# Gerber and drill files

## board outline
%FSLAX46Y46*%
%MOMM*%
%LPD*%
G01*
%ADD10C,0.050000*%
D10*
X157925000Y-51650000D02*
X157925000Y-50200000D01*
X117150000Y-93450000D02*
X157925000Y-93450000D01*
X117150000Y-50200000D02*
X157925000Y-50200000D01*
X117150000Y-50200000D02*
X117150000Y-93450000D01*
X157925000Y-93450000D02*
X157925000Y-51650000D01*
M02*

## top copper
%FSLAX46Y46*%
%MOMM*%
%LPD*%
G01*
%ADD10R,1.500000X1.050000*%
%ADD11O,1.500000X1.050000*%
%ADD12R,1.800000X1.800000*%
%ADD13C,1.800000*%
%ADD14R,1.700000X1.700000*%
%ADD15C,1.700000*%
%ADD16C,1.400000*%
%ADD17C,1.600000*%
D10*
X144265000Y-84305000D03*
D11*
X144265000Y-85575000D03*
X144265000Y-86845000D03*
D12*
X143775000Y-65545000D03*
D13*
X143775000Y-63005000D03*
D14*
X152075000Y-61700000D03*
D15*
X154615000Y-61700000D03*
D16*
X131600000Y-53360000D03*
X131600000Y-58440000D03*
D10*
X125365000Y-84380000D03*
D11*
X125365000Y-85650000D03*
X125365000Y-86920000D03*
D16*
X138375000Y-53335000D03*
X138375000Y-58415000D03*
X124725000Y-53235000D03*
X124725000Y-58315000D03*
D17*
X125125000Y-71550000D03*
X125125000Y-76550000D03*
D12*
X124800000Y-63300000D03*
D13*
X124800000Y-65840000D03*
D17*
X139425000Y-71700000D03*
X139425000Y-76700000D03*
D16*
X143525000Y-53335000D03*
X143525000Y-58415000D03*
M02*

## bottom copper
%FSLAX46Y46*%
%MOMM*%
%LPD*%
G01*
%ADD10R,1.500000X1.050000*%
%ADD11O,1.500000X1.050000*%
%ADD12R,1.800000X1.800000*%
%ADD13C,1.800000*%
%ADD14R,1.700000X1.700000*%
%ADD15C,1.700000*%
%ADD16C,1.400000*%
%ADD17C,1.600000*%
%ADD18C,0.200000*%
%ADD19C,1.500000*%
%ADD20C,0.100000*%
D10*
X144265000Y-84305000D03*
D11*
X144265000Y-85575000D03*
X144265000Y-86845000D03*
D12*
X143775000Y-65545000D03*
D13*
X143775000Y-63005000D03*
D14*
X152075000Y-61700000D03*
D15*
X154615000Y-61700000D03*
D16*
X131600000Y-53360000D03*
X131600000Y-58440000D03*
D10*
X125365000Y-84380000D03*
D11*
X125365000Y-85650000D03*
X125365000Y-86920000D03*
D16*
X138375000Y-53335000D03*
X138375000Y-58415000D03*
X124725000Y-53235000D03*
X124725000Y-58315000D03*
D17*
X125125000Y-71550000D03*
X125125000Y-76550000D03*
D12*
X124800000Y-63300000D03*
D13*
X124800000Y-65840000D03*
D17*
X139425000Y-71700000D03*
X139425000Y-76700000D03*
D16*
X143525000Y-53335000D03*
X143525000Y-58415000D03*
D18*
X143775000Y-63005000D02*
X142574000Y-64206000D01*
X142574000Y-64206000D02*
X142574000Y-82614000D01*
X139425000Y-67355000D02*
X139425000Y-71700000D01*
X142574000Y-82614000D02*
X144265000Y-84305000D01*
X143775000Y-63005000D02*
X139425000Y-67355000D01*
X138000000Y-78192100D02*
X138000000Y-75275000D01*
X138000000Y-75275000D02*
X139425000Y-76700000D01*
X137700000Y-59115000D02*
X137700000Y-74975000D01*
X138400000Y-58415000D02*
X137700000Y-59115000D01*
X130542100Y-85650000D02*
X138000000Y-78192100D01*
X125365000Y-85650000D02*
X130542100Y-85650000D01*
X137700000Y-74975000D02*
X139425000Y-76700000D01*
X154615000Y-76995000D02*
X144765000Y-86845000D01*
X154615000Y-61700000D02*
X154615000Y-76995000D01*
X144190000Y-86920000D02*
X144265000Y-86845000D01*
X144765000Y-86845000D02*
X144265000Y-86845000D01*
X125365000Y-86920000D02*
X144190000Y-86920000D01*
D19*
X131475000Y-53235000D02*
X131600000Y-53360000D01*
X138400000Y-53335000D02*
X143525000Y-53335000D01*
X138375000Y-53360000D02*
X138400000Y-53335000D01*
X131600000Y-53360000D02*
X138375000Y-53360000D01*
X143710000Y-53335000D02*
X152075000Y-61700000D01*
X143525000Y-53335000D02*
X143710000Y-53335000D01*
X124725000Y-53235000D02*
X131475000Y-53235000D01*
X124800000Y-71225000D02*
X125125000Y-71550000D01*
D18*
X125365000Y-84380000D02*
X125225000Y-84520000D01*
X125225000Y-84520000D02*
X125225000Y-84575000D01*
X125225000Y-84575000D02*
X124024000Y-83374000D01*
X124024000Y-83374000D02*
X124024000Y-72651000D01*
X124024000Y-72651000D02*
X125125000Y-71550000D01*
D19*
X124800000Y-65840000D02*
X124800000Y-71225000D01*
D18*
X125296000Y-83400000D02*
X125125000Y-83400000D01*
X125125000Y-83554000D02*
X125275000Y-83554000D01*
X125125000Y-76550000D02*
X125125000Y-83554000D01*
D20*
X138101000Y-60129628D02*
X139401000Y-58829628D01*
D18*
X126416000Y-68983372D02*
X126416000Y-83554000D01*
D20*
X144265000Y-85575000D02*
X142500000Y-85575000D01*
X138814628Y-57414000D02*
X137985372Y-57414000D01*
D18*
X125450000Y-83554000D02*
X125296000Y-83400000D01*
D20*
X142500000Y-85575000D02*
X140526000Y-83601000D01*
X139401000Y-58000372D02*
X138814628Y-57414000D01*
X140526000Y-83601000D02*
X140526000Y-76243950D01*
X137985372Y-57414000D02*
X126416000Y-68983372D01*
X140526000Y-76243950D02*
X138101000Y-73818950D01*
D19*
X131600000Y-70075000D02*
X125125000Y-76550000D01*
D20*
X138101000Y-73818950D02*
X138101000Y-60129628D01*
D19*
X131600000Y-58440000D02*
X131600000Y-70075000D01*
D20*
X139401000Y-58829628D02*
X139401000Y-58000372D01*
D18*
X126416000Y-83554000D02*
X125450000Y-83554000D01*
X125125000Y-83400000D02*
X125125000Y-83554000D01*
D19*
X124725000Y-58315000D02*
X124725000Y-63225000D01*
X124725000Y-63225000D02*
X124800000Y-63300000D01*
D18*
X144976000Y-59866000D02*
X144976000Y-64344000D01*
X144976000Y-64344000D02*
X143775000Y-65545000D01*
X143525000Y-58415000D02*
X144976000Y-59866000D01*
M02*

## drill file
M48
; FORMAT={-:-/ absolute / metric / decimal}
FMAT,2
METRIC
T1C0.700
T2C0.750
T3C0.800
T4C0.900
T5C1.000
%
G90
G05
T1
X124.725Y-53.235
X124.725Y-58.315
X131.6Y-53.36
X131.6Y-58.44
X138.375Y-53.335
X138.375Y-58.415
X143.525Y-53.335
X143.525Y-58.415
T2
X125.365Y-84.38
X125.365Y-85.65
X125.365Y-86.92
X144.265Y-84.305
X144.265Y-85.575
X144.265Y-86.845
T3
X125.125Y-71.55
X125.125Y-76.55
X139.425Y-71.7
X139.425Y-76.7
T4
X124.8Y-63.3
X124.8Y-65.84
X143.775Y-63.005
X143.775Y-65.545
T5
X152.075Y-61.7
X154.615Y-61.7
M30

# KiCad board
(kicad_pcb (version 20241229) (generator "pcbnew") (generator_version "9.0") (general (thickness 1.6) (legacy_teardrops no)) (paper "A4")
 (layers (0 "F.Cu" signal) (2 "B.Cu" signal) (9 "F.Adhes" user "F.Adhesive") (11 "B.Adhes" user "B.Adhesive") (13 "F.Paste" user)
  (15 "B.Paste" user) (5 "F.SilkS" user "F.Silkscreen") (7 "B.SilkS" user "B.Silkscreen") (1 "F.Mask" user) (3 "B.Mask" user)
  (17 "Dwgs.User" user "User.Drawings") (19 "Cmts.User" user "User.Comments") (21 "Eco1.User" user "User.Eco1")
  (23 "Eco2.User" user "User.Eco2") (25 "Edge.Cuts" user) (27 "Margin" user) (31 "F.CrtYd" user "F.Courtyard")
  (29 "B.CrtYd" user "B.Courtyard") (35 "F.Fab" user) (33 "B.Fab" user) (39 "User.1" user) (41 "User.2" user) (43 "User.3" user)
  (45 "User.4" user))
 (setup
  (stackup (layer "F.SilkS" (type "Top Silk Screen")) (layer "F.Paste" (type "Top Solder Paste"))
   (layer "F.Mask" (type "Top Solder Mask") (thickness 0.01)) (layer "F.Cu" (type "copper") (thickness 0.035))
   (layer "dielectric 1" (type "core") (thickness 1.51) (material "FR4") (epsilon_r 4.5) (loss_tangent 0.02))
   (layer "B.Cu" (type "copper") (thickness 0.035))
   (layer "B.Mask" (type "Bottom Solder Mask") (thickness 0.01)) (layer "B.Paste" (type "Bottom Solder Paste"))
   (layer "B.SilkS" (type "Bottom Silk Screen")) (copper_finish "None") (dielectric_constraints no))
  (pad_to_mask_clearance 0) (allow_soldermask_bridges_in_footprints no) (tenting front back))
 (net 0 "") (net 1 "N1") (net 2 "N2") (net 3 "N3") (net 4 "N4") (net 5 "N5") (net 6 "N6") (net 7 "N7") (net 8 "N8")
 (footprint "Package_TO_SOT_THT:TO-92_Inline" (layer "F.Cu") (at 144.265 84.305 -90)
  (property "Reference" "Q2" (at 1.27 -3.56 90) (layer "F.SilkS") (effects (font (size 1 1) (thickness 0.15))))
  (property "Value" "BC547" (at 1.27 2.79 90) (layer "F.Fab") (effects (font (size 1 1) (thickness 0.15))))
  (pad "1" thru_hole rect (at 0 0 270) (size 1.05 1.5) (drill 0.75) (layers "*.Cu" "*.Mask") (remove_unused_layers no) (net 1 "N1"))
  (pad "2" thru_hole oval (at 1.27 0 270) (size 1.05 1.5) (drill 0.75) (layers "*.Cu" "*.Mask") (remove_unused_layers no) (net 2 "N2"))
  (pad "3" thru_hole oval (at 2.54 0 270) (size 1.05 1.5) (drill 0.75) (layers "*.Cu" "*.Mask") (remove_unused_layers no) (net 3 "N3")))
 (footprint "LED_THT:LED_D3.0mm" (layer "F.Cu") (at 143.775 65.545 90)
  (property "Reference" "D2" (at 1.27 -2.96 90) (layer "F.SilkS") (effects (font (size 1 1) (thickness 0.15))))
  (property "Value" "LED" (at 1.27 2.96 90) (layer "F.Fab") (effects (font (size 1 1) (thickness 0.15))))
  (pad "1" thru_hole rect (at 0 0 90) (size 1.8 1.8) (drill 0.9) (layers "*.Cu" "*.Mask") (remove_unused_layers no) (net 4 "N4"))
  (pad "2" thru_hole circle (at 2.54 0 90) (size 1.8 1.8) (drill 0.9) (layers "*.Cu" "*.Mask") (remove_unused_layers no) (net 1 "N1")))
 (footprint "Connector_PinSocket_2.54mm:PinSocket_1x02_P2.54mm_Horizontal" (layer "F.Cu") (at 152.075 61.7 90)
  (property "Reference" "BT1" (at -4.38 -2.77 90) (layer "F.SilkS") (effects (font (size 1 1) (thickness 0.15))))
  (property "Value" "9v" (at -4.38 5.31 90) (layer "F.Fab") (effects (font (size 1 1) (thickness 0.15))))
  (pad "1" thru_hole rect (at 0 0 90) (size 1.7 1.7) (drill 1) (layers "*.Cu" "*.Mask") (remove_unused_layers no) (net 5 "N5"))
  (pad "2" thru_hole circle (at 0 2.54 90) (size 1.7 1.7) (drill 1) (layers "*.Cu" "*.Mask") (remove_unused_layers no) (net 3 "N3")))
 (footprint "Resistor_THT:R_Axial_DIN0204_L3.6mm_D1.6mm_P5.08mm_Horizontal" (layer "F.Cu") (at 131.6 53.36 -90)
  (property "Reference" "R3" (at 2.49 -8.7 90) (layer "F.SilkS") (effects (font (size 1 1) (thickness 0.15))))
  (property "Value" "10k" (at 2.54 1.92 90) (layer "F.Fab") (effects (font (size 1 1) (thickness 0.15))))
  (pad "1" thru_hole circle (at 0 0 270) (size 1.4 1.4) (drill 0.7) (layers "*.Cu" "*.Mask") (remove_unused_layers no) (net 5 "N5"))
  (pad "2" thru_hole circle (at 5.08 0 270) (size 1.4 1.4) (drill 0.7) (layers "*.Cu" "*.Mask") (remove_unused_layers no) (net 2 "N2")))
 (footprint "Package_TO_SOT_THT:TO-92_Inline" (layer "F.Cu") (at 125.365 84.38 -90)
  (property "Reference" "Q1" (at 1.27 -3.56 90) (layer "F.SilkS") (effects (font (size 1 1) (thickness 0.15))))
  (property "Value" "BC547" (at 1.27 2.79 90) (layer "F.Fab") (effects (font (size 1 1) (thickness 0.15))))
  (pad "1" thru_hole rect (at 0 0 270) (size 1.05 1.5) (drill 0.75) (layers "*.Cu" "*.Mask") (remove_unused_layers no) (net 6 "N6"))
  (pad "2" thru_hole oval (at 1.27 0 270) (size 1.05 1.5) (drill 0.75) (layers "*.Cu" "*.Mask") (remove_unused_layers no) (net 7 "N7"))
  (pad "3" thru_hole oval (at 2.54 0 270) (size 1.05 1.5) (drill 0.75) (layers "*.Cu" "*.Mask") (remove_unused_layers no) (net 3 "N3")))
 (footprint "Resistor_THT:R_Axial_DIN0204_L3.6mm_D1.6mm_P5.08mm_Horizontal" (layer "F.Cu") (at 138.375 53.335 -90)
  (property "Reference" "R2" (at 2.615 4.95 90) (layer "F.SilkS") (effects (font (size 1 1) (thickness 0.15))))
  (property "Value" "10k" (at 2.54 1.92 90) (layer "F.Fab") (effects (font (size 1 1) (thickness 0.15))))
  (pad "1" thru_hole circle (at 0 0 270) (size 1.4 1.4) (drill 0.7) (layers "*.Cu" "*.Mask") (remove_unused_layers no) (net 5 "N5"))
  (pad "2" thru_hole circle (at 5.08 0 270) (size 1.4 1.4) (drill 0.7) (layers "*.Cu" "*.Mask") (remove_unused_layers no) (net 7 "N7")))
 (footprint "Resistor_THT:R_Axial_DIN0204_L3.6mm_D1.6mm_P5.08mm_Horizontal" (layer "F.Cu") (at 124.725 53.235 -90)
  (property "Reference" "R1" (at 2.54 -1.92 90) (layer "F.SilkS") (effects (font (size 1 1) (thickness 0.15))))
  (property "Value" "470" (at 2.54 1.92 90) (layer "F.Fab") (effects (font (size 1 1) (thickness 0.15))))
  (pad "1" thru_hole circle (at 0 0 270) (size 1.4 1.4) (drill 0.7) (layers "*.Cu" "*.Mask") (remove_unused_layers no) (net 5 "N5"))
  (pad "2" thru_hole circle (at 5.08 0 270) (size 1.4 1.4) (drill 0.7) (layers "*.Cu" "*.Mask") (remove_unused_layers no) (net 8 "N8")))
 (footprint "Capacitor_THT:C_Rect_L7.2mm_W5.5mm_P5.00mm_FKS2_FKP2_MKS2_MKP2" (layer "F.Cu") (at 125.125 71.55 -90)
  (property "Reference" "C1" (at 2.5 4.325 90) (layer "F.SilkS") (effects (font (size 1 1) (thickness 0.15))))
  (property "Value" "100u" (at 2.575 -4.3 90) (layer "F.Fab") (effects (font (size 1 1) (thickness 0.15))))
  (pad "1" thru_hole circle (at 0 0 270) (size 1.6 1.6) (drill 0.8) (layers "*.Cu" "*.Mask") (remove_unused_layers no) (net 6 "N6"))
  (pad "2" thru_hole circle (at 5 0 270) (size 1.6 1.6) (drill 0.8) (layers "*.Cu" "*.Mask") (remove_unused_layers no) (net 2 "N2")))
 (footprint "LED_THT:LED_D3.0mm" (layer "F.Cu") (at 124.8 63.3 -90)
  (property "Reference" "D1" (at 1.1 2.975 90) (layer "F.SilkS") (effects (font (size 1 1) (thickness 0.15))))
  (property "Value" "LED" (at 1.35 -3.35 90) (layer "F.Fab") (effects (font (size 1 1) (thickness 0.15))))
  (pad "1" thru_hole rect (at 0 0 270) (size 1.8 1.8) (drill 0.9) (layers "*.Cu" "*.Mask") (remove_unused_layers no) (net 8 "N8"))
  (pad "2" thru_hole circle (at 2.54 0 270) (size 1.8 1.8) (drill 0.9) (layers "*.Cu" "*.Mask") (remove_unused_layers no) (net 6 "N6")))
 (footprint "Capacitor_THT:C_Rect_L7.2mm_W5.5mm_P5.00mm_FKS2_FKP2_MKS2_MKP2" (layer "F.Cu") (at 139.425 71.7 -90)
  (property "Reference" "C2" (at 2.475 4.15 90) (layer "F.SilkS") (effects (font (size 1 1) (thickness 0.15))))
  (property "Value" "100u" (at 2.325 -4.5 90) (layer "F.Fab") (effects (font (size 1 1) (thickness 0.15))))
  (pad "1" thru_hole circle (at 0 0 270) (size 1.6 1.6) (drill 0.8) (layers "*.Cu" "*.Mask") (remove_unused_layers no) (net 1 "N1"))
  (pad "2" thru_hole circle (at 5 0 270) (size 1.6 1.6) (drill 0.8) (layers "*.Cu" "*.Mask") (remove_unused_layers no) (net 7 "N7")))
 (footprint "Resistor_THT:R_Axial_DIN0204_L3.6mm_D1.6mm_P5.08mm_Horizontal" (layer "F.Cu") (at 143.525 53.335 -90)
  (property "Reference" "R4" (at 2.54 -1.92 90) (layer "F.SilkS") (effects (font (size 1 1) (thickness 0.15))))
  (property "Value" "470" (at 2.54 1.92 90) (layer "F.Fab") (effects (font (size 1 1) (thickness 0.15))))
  (pad "1" thru_hole circle (at 0 0 270) (size 1.4 1.4) (drill 0.7) (layers "*.Cu" "*.Mask") (remove_unused_layers no) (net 5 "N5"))
  (pad "2" thru_hole circle (at 5.08 0 270) (size 1.4 1.4) (drill 0.7) (layers "*.Cu" "*.Mask") (remove_unused_layers no) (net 4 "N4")))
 (gr_line (start 157.925 51.65) (end 157.925 50.2) (stroke (width 0.05) (type default)) (layer "Edge.Cuts"))
 (gr_line (start 117.15 93.45) (end 157.925 93.45) (stroke (width 0.05) (type default)) (layer "Edge.Cuts"))
 (gr_line (start 117.15 50.2) (end 157.925 50.2) (stroke (width 0.05) (type default)) (layer "Edge.Cuts"))
 (gr_line (start 117.15 50.2) (end 117.15 93.45) (stroke (width 0.05) (type default)) (layer "Edge.Cuts"))
 (gr_line (start 157.925 93.45) (end 157.925 51.65) (stroke (width 0.05) (type default)) (layer "Edge.Cuts"))
 (segment (start 143.775 63.005) (end 142.574 64.206) (width 0.2) (layer "B.Cu") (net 1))
 (segment (start 142.574 64.206) (end 142.574 82.614) (width 0.2) (layer "B.Cu") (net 1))
 (segment (start 139.425 67.355) (end 139.425 71.7) (width 0.2) (layer "B.Cu") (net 1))
 (segment (start 142.574 82.614) (end 144.265 84.305) (width 0.2) (layer "B.Cu") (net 1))
 (segment (start 143.775 63.005) (end 139.425 67.355) (width 0.2) (layer "B.Cu") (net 1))
 (segment (start 138 78.1921) (end 138 75.275) (width 0.2) (layer "B.Cu") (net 7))
 (segment (start 138 75.275) (end 139.425 76.7) (width 0.2) (layer "B.Cu") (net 7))
 (segment (start 137.7 59.115) (end 137.7 74.975) (width 0.2) (layer "B.Cu") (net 7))
 (segment (start 138.4 58.415) (end 137.7 59.115) (width 0.2) (layer "B.Cu") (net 7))
 (segment (start 130.5421 85.65) (end 138 78.1921) (width 0.2) (layer "B.Cu") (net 7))
 (segment (start 125.365 85.65) (end 130.5421 85.65) (width 0.2) (layer "B.Cu") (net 7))
 (segment (start 137.7 74.975) (end 139.425 76.7) (width 0.2) (layer "B.Cu") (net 7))
 (segment (start 154.615 76.995) (end 144.765 86.845) (width 0.2) (layer "B.Cu") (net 3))
 (segment (start 154.615 61.7) (end 154.615 76.995) (width 0.2) (layer "B.Cu") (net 3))
 (segment (start 144.19 86.92) (end 144.265 86.845) (width 0.2) (layer "B.Cu") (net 3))
 (segment (start 144.765 86.845) (end 144.265 86.845) (width 0.2) (layer "B.Cu") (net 3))
 (segment (start 125.365 86.92) (end 144.19 86.92) (width 0.2) (layer "B.Cu") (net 3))
 (segment (start 131.475 53.235) (end 131.6 53.36) (width 1.5) (layer "B.Cu") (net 5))
 (segment (start 138.4 53.335) (end 143.525 53.335) (width 1.5) (layer "B.Cu") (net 5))
 (segment (start 138.375 53.36) (end 138.4 53.335) (width 1.5) (layer "B.Cu") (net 5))
 (segment (start 131.6 53.36) (end 138.375 53.36) (width 1.5) (layer "B.Cu") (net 5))
 (segment (start 143.71 53.335) (end 152.075 61.7) (width 1.5) (layer "B.Cu") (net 5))
 (segment (start 143.525 53.335) (end 143.71 53.335) (width 1.5) (layer "B.Cu") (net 5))
 (segment (start 124.725 53.235) (end 131.475 53.235) (width 1.5) (layer "B.Cu") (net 5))
 (segment (start 124.8 71.225) (end 125.125 71.55) (width 1.5) (layer "B.Cu") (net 6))
 (segment (start 125.365 84.38) (end 125.225 84.52) (width 0.2) (layer "B.Cu") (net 6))
 (segment (start 125.225 84.52) (end 125.225 84.575) (width 0.2) (layer "B.Cu") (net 6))
 (segment (start 125.225 84.575) (end 124.024 83.374) (width 0.2) (layer "B.Cu") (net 6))
 (segment (start 124.024 83.374) (end 124.024 72.651) (width 0.2) (layer "B.Cu") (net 6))
 (segment (start 124.024 72.651) (end 125.125 71.55) (width 0.2) (layer "B.Cu") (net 6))
 (segment (start 124.8 65.84) (end 124.8 71.225) (width 1.5) (layer "B.Cu") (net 6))
 (segment (start 125.296 83.4) (end 125.125 83.4) (width 0.2) (layer "B.Cu") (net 2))
 (segment (start 125.125 83.554) (end 125.275 83.554) (width 0.2) (layer "B.Cu") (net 2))
 (segment (start 125.125 76.55) (end 125.125 83.554) (width 0.2) (layer "B.Cu") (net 2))
 (segment (start 138.101 60.129628) (end 139.401 58.829628) (width 0.1) (layer "B.Cu") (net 2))
 (segment (start 126.416 68.983372) (end 126.416 83.554) (width 0.2) (layer "B.Cu") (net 2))
 (segment (start 144.265 85.575) (end 142.5 85.575) (width 0.1) (layer "B.Cu") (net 2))
 (segment (start 138.814628 57.414) (end 137.985372 57.414) (width 0.1) (layer "B.Cu") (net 2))
 (segment (start 125.45 83.554) (end 125.296 83.4) (width 0.2) (layer "B.Cu") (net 2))
 (segment (start 142.5 85.575) (end 140.526 83.601) (width 0.1) (layer "B.Cu") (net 2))
 (segment (start 139.401 58.000372) (end 138.814628 57.414) (width 0.1) (layer "B.Cu") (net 2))
 (segment (start 140.526 83.601) (end 140.526 76.24395) (width 0.1) (layer "B.Cu") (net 2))
 (segment (start 137.985372 57.414) (end 126.416 68.983372) (width 0.1) (layer "B.Cu") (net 2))
 (segment (start 140.526 76.24395) (end 138.101 73.81895) (width 0.1) (layer "B.Cu") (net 2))
 (segment (start 131.6 70.075) (end 125.125 76.55) (width 1.5) (layer "B.Cu") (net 2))
 (segment (start 138.101 73.81895) (end 138.101 60.129628) (width 0.1) (layer "B.Cu") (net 2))
 (segment (start 131.6 58.44) (end 131.6 70.075) (width 1.5) (layer "B.Cu") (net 2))
 (segment (start 139.401 58.829628) (end 139.401 58.000372) (width 0.1) (layer "B.Cu") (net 2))
 (segment (start 126.416 83.554) (end 125.45 83.554) (width 0.2) (layer "B.Cu") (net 2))
 (segment (start 125.125 83.4) (end 125.125 83.554) (width 0.2) (layer "B.Cu") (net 2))
 (segment (start 124.725 58.315) (end 124.725 63.225) (width 1.5) (layer "B.Cu") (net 8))
 (segment (start 124.725 63.225) (end 124.8 63.3) (width 1.5) (layer "B.Cu") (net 8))
 (segment (start 144.976 59.866) (end 144.976 64.344) (width 0.2) (layer "B.Cu") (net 4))
 (segment (start 144.976 64.344) (end 143.775 65.545) (width 0.2) (layer "B.Cu") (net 4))
 (segment (start 143.525 58.415) (end 144.976 59.866) (width 0.2) (layer "B.Cu") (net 4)))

